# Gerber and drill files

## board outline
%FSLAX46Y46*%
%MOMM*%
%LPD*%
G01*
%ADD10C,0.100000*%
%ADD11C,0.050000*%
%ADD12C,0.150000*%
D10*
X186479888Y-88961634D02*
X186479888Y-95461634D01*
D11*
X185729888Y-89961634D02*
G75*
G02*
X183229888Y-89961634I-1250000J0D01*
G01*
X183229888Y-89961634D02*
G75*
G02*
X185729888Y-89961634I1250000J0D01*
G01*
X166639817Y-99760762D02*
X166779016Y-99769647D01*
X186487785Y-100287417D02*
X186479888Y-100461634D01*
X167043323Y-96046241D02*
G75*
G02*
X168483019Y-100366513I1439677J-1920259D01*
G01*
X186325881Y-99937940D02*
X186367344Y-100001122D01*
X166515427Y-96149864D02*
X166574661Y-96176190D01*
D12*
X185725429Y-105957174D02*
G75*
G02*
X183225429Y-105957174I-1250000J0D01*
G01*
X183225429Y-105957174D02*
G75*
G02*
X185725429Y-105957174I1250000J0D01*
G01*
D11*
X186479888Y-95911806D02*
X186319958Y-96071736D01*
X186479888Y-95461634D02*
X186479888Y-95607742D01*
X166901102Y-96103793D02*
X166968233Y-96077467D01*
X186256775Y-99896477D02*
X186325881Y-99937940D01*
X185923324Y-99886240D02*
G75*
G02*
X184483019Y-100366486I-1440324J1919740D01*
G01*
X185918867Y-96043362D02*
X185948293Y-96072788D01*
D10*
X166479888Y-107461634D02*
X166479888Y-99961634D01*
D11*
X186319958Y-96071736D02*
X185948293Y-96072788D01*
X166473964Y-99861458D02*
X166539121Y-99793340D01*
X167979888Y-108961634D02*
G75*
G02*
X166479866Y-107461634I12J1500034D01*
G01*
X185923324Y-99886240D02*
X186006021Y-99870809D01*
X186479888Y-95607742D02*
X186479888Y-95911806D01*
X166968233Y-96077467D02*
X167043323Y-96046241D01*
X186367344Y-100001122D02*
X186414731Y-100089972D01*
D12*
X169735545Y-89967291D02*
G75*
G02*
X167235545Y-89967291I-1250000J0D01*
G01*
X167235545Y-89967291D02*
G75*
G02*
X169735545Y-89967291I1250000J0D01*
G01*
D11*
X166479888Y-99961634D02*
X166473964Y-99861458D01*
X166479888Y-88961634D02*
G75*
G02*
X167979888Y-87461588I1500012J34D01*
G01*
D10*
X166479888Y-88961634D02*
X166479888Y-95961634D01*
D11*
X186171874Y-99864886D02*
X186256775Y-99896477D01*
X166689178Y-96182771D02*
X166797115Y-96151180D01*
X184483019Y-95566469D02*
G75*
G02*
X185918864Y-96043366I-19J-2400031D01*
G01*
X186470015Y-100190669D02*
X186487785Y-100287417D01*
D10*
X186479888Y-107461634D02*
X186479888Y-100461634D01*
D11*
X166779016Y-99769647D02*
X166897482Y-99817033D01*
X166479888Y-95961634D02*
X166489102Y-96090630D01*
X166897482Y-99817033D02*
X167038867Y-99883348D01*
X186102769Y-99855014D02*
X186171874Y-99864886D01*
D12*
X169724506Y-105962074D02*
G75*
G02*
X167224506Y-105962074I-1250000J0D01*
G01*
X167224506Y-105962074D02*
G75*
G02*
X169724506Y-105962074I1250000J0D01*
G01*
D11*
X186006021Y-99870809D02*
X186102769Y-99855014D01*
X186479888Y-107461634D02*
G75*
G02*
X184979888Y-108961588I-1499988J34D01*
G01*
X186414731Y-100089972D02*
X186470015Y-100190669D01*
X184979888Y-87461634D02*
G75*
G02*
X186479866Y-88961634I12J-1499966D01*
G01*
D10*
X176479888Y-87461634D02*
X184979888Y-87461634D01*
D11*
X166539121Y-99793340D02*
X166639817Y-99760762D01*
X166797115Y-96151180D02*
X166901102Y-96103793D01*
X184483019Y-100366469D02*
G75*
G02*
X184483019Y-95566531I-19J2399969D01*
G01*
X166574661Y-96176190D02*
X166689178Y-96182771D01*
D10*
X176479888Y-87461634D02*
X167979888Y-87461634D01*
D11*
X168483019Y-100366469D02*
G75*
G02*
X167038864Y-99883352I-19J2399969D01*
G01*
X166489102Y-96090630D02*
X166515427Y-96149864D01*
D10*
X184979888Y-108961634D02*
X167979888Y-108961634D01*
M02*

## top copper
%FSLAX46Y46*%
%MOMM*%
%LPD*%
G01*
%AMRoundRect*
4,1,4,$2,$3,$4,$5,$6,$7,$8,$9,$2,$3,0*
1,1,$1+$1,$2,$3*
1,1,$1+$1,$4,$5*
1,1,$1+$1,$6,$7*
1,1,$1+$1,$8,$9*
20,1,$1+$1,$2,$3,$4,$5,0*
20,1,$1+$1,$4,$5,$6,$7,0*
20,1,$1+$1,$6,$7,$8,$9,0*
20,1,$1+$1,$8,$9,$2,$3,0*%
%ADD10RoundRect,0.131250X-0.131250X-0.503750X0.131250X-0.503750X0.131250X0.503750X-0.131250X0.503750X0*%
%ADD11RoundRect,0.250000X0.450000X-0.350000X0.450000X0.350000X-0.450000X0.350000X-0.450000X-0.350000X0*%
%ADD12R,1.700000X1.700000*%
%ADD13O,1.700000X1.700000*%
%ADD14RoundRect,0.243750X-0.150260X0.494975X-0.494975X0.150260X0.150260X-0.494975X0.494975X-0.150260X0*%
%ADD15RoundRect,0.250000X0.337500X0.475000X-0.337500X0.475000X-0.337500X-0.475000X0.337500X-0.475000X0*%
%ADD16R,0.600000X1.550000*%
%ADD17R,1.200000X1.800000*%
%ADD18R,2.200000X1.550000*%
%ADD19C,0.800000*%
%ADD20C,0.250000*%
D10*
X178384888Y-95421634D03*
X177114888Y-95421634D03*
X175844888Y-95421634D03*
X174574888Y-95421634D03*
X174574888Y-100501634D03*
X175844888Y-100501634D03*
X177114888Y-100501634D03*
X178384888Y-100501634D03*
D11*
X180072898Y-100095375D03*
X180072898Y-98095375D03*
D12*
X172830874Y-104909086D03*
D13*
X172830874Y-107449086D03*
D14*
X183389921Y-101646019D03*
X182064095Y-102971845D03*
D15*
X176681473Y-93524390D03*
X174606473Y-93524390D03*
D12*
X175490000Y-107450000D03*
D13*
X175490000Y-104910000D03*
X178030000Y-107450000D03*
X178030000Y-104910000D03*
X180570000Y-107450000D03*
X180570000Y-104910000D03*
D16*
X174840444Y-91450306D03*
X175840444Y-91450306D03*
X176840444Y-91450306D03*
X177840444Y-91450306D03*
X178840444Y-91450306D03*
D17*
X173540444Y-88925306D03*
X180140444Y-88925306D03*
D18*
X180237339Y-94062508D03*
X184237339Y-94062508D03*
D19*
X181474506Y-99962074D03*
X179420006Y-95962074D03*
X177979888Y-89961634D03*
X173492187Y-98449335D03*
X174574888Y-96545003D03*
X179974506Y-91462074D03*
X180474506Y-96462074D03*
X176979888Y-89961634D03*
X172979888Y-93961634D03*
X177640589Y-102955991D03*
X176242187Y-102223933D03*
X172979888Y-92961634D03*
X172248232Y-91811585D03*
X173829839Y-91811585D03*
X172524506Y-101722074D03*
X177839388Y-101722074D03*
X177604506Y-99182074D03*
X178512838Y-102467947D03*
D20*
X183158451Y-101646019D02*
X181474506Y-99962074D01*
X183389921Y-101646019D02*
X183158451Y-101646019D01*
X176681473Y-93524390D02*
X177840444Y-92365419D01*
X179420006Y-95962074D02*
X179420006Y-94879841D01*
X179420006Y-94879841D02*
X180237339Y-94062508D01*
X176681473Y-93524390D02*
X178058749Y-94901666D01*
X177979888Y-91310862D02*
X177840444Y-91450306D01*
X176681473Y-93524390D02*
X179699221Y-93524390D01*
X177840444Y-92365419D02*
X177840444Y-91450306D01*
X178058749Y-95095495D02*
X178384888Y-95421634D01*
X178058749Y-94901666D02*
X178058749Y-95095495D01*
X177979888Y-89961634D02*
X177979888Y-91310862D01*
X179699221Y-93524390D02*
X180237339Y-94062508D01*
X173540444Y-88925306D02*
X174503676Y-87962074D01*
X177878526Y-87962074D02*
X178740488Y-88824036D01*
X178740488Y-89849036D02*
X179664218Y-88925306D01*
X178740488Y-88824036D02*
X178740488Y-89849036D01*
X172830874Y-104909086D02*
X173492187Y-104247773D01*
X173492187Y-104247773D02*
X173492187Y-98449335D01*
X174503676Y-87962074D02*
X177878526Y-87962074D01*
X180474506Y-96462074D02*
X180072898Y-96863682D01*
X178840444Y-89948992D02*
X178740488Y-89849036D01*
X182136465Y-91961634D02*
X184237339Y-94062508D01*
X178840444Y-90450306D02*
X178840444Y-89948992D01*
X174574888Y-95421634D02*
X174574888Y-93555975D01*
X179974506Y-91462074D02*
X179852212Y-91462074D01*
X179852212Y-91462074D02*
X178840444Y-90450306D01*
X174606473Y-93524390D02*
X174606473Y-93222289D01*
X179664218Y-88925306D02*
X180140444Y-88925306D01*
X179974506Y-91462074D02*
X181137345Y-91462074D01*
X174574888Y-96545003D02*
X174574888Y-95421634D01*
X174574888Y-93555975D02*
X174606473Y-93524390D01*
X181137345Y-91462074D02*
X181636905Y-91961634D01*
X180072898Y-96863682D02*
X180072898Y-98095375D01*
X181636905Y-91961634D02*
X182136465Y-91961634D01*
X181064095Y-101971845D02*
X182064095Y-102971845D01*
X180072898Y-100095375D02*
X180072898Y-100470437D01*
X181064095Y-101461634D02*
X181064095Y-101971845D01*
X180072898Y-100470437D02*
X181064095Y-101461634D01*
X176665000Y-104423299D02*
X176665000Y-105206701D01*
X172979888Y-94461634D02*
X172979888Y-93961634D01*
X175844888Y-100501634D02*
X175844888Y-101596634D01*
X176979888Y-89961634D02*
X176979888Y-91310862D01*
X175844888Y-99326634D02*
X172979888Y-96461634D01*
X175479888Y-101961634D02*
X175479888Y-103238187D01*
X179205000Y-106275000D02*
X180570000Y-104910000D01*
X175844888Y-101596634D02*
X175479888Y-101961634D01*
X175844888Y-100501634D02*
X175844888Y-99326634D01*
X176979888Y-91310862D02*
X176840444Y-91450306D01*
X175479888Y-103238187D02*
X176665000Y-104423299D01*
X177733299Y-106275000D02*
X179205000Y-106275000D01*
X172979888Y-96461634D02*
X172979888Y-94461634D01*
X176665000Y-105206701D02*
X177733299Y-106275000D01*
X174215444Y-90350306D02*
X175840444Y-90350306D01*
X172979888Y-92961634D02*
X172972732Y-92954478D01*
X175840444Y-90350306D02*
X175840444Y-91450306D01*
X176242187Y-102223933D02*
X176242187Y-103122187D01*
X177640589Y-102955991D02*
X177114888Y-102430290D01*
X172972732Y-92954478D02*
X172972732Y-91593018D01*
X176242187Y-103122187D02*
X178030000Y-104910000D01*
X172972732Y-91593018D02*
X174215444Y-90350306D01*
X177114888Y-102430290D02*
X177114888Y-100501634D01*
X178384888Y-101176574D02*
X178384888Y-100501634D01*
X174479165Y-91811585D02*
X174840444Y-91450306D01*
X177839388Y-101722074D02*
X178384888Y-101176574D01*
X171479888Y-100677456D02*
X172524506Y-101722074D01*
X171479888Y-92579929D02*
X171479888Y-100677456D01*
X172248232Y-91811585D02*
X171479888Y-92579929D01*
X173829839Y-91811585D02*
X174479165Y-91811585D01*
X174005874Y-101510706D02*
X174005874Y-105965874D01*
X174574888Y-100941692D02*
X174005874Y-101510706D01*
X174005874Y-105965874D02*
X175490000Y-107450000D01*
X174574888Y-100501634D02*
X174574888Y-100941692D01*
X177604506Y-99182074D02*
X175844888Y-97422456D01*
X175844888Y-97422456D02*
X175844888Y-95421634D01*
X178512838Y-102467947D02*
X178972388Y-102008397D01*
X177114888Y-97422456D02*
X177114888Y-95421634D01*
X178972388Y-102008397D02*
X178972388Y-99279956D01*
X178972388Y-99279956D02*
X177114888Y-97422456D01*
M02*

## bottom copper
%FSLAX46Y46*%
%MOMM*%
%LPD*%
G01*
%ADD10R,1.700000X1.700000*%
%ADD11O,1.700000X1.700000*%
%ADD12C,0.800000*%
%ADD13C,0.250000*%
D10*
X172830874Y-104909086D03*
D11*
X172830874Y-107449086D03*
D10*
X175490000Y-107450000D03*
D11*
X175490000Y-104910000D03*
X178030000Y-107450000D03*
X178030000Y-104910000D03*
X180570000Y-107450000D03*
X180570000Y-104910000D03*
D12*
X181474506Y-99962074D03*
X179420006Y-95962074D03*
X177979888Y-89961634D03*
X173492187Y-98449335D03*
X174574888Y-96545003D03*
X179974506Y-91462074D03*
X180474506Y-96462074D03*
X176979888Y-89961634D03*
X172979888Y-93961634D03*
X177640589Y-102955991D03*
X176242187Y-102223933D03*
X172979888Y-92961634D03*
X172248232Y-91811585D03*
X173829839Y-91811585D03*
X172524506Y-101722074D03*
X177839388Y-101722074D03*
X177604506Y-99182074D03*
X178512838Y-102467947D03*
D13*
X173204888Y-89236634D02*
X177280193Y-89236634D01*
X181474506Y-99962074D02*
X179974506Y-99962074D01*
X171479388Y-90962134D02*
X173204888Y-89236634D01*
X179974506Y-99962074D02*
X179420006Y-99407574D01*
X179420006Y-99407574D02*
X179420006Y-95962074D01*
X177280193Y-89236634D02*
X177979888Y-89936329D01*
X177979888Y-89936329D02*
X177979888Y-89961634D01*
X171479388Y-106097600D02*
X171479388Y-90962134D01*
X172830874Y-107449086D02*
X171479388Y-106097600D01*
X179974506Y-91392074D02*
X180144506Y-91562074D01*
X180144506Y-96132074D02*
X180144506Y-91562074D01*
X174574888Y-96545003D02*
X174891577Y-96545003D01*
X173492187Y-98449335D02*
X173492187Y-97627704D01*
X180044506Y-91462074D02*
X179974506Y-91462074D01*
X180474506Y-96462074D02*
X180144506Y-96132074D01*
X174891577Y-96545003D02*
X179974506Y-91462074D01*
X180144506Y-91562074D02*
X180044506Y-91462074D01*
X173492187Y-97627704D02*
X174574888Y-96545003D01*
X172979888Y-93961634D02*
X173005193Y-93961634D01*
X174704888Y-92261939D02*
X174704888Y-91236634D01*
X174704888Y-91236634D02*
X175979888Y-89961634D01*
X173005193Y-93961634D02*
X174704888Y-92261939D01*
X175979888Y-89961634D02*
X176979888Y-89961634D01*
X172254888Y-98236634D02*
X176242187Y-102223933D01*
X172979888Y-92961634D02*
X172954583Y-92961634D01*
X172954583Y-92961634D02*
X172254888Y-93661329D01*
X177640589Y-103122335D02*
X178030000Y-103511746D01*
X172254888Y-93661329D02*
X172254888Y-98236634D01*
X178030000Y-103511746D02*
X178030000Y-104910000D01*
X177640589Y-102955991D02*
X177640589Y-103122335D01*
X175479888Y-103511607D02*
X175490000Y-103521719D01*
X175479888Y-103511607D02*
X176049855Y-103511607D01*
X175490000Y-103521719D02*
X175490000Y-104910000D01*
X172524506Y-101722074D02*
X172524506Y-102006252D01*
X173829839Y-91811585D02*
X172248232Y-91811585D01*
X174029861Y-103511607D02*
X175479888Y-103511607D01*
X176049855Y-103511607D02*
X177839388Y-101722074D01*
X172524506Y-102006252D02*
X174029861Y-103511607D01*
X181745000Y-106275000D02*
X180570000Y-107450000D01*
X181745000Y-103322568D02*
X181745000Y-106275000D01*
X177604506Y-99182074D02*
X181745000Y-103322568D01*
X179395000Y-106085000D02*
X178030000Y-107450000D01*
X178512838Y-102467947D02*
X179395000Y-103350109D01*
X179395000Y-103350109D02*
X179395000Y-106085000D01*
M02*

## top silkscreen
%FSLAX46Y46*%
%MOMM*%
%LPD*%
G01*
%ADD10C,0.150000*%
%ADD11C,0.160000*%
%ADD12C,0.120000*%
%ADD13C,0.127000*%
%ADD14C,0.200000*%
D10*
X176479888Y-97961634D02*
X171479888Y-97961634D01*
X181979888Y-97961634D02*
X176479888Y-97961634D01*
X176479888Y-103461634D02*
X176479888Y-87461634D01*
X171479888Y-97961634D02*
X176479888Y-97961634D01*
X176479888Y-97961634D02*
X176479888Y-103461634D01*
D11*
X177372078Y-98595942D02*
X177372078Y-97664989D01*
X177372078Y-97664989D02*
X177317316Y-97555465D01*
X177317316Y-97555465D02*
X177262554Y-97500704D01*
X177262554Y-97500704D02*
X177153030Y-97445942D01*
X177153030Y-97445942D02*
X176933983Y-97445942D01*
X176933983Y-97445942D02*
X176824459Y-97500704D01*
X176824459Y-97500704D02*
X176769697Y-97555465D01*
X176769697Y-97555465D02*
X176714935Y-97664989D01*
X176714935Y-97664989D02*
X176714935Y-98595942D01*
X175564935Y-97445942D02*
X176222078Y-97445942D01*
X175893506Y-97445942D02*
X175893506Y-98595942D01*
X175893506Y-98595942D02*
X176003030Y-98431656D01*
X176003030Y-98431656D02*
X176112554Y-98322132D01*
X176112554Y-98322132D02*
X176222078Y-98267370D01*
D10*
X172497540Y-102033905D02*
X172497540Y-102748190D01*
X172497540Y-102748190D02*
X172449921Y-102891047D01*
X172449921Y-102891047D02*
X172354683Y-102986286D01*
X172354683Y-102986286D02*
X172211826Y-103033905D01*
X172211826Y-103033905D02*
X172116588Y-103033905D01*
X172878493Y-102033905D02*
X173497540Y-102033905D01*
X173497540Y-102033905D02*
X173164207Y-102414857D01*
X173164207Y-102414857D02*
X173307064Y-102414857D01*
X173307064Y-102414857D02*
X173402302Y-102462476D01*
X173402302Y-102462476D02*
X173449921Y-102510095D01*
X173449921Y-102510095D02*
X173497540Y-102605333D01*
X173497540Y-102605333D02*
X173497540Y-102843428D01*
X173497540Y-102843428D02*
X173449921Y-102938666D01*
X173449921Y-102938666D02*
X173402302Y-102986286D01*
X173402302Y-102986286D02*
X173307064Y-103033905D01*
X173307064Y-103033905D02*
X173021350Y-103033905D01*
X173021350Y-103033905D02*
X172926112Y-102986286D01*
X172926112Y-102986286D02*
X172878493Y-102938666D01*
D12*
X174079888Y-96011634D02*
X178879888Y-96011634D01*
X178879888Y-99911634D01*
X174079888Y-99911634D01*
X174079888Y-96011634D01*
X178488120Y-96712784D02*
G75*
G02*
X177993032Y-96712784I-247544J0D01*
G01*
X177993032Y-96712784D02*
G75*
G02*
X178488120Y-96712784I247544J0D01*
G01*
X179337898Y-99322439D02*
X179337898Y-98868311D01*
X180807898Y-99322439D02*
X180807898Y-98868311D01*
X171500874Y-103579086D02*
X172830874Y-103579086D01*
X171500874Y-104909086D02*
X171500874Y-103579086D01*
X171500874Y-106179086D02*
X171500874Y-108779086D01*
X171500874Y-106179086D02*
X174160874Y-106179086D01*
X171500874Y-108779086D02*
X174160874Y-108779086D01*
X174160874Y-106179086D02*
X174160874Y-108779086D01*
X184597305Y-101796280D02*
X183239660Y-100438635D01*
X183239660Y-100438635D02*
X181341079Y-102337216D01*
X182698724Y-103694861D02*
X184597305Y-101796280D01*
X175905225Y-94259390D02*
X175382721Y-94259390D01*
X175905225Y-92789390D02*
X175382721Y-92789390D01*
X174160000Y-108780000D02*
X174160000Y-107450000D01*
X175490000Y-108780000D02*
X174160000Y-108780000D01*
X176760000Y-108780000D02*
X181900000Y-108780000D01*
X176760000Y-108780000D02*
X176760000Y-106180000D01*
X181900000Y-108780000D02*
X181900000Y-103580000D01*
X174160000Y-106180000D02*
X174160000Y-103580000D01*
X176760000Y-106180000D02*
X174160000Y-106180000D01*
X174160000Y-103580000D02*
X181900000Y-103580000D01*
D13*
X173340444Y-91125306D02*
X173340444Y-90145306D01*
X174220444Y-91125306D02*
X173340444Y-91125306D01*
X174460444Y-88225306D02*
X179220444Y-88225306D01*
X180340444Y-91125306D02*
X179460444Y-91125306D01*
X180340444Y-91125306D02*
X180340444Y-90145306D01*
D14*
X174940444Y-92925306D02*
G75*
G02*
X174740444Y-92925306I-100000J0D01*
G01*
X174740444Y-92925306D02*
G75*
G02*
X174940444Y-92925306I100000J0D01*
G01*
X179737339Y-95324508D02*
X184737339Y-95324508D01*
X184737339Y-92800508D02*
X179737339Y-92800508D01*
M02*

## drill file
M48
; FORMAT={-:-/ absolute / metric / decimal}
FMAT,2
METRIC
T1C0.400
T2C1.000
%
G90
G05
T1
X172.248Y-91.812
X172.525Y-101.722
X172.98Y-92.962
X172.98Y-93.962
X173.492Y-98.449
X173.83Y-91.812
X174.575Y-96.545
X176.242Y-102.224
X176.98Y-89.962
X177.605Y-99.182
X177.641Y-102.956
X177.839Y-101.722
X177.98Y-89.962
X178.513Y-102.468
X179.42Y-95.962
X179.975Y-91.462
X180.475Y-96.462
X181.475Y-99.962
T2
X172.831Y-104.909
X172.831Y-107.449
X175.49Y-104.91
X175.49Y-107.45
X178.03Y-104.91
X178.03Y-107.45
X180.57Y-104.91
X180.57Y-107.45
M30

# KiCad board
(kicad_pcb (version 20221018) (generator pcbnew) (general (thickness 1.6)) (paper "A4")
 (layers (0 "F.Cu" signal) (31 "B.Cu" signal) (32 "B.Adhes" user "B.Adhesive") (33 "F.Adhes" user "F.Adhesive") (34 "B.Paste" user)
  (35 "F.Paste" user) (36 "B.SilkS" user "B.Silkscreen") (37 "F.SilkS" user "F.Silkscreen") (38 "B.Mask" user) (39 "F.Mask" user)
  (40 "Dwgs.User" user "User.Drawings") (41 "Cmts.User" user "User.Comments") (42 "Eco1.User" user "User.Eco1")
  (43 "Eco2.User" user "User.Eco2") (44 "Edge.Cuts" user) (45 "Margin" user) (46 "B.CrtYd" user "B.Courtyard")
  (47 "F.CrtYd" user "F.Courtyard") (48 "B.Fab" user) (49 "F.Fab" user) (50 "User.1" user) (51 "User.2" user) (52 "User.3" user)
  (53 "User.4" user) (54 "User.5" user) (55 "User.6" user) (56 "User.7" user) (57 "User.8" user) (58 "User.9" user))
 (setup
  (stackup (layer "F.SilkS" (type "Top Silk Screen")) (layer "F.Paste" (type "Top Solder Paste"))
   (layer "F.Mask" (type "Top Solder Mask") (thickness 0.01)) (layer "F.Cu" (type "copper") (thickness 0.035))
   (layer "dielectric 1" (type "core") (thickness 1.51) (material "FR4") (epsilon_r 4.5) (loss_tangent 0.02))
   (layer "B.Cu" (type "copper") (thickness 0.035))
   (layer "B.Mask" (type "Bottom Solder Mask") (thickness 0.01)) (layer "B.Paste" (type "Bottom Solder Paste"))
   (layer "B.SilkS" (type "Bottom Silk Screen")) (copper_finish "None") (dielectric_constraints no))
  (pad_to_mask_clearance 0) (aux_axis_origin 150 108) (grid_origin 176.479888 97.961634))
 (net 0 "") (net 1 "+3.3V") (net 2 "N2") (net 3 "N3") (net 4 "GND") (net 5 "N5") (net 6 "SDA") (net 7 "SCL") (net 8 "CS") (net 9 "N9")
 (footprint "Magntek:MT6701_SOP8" (layer "F.Cu") (at 176.479888 97.961634 180)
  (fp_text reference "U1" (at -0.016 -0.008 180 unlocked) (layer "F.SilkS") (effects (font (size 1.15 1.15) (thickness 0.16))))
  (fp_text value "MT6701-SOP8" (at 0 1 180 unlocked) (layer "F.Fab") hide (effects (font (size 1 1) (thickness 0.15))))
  (fp_rect (start -2.4 -1.95) (end 2.4 1.95) (stroke (width 0.12) (type default)) (fill none) (layer "F.SilkS"))
  (fp_circle (center -1.760688 1.24885) (end -1.598307 1.435694) (stroke (width 0.12) (type default)) (fill none) (layer "F.SilkS"))
  (pad "1" smd roundrect (at -1.905 2.54) (size 0.525 1.27) (layers "F.Cu" "F.Paste" "F.Mask") (roundrect_rratio 0.25) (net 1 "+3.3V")
   (thermal_bridge_angle 45))
  (pad "2" smd roundrect (at -0.635 2.54) (size 0.525 1.27) (layers "F.Cu" "F.Paste" "F.Mask") (roundrect_rratio 0.25) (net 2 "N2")
   (thermal_bridge_angle 45))
  (pad "3" smd roundrect (at 0.635 2.54) (size 0.525 1.27) (layers "F.Cu" "F.Paste" "F.Mask") (roundrect_rratio 0.25) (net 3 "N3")
   (thermal_bridge_angle 45))
  (pad "4" smd roundrect (at 1.905 2.54) (size 0.525 1.27) (layers "F.Cu" "F.Paste" "F.Mask") (roundrect_rratio 0.25) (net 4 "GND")
   (thermal_bridge_angle 45))
  (pad "5" smd roundrect (at 1.905 -2.54) (size 0.525 1.27) (layers "F.Cu" "F.Paste" "F.Mask") (roundrect_rratio 0.25) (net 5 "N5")
   (thermal_bridge_angle 45))
  (pad "6" smd roundrect (at 0.635 -2.54) (size 0.525 1.27) (layers "F.Cu" "F.Paste" "F.Mask") (roundrect_rratio 0.25) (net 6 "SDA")
   (thermal_bridge_angle 45))
  (pad "7" smd roundrect (at -0.635 -2.54) (size 0.525 1.27) (layers "F.Cu" "F.Paste" "F.Mask") (roundrect_rratio 0.25) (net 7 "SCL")
   (thermal_bridge_angle 45))
  (pad "8" smd roundrect (at -1.905 -2.54) (size 0.525 1.27) (layers "F.Cu" "F.Paste" "F.Mask") (roundrect_rratio 0.25) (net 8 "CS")
   (thermal_bridge_angle 45)))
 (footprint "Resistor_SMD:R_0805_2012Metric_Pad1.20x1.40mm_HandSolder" (layer "F.Cu") (at 180.072898 99.095375 90)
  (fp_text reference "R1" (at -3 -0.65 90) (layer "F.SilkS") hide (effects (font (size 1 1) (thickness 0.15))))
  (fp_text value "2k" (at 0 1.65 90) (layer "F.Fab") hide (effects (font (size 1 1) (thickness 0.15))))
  (fp_line (start -0.227064 -0.735) (end 0.227064 -0.735) (stroke (width 0.12) (type solid)) (layer "F.SilkS"))
  (fp_line (start -0.227064 0.735) (end 0.227064 0.735) (stroke (width 0.12) (type solid)) (layer "F.SilkS"))
  (pad "1" smd roundrect (at -1 0 90) (size 1.2 1.4) (layers "F.Cu" "F.Paste" "F.Mask") (roundrect_rratio 0.208333) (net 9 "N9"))
  (pad "2" smd roundrect (at 1 0 90) (size 1.2 1.4) (layers "F.Cu" "F.Paste" "F.Mask") (roundrect_rratio 0.208333) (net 4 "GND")))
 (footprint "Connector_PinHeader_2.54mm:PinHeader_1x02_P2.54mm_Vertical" (layer "F.Cu") (at 172.830874 104.909086)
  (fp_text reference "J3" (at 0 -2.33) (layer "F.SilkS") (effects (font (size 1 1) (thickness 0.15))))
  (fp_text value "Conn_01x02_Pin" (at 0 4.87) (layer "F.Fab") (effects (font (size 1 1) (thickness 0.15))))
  (fp_line (start -1.33 -1.33) (end 0 -1.33) (stroke (width 0.12) (type solid)) (layer "F.SilkS"))
  (fp_line (start -1.33 0) (end -1.33 -1.33) (stroke (width 0.12) (type solid)) (layer "F.SilkS"))
  (fp_line (start -1.33 1.27) (end -1.33 3.87) (stroke (width 0.12) (type solid)) (layer "F.SilkS"))
  (fp_line (start -1.33 1.27) (end 1.33 1.27) (stroke (width 0.12) (type solid)) (layer "F.SilkS"))
  (fp_line (start -1.33 3.87) (end 1.33 3.87) (stroke (width 0.12) (type solid)) (layer "F.SilkS"))
  (fp_line (start 1.33 1.27) (end 1.33 3.87) (stroke (width 0.12) (type solid)) (layer "F.SilkS"))
  (pad "1" thru_hole rect (at 0 0) (size 1.7 1.7) (drill 1) (layers "*.Cu" "*.Mask") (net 4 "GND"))
  (pad "2" thru_hole oval (at 0 2.54) (size 1.7 1.7) (drill 1) (layers "*.Cu" "*.Mask") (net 1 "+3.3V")))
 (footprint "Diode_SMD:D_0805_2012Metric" (layer "F.Cu") (at 182.727008 102.308932 -135)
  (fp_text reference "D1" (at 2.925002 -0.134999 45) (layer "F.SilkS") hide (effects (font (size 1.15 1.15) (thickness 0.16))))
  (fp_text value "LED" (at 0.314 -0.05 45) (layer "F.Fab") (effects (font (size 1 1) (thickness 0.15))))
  (fp_line (start -1.685 -0.96) (end -1.685 0.96) (stroke (width 0.12) (type solid)) (layer "F.SilkS"))
  (fp_line (start -1.685 0.96) (end 1 0.96) (stroke (width 0.12) (type solid)) (layer "F.SilkS"))
  (fp_line (start 1 -0.96) (end -1.685 -0.96) (stroke (width 0.12) (type solid)) (layer "F.SilkS"))
  (pad "1" smd roundrect (at -0.9375 0 225) (size 0.975 1.4) (layers "F.Cu" "F.Paste" "F.Mask") (roundrect_rratio 0.25) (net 1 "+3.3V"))
  (pad "2" smd roundrect (at 0.9375 0 225) (size 0.975 1.4) (layers "F.Cu" "F.Paste" "F.Mask") (roundrect_rratio 0.25) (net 9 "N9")))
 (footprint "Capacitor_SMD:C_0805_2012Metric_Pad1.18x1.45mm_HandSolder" (layer "F.Cu") (at 175.643973 93.52439 180)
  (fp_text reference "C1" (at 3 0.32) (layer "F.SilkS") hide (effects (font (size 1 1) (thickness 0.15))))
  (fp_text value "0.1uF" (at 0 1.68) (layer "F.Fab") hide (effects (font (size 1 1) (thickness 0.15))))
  (fp_line (start -0.261252 -0.735) (end 0.261252 -0.735) (stroke (width 0.12) (type solid)) (layer "F.SilkS"))
  (fp_line (start -0.261252 0.735) (end 0.261252 0.735) (stroke (width 0.12) (type solid)) (layer "F.SilkS"))
  (pad "1" smd roundrect (at -1.0375 0 180) (size 1.175 1.45) (layers "F.Cu" "F.Paste" "F.Mask") (roundrect_rratio 0.212766) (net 1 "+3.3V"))
  (pad "2" smd roundrect (at 1.0375 0 180) (size 1.175 1.45) (layers "F.Cu" "F.Paste" "F.Mask") (roundrect_rratio 0.212766) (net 4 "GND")))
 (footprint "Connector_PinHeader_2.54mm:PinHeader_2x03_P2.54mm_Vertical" (layer "F.Cu") (at 175.49 107.45 90)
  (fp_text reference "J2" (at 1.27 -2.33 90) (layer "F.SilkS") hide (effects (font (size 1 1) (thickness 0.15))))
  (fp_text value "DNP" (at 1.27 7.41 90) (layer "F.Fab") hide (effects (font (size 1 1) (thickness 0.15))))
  (fp_line (start -1.33 -1.33) (end 0 -1.33) (stroke (width 0.12) (type solid)) (layer "F.SilkS"))
  (fp_line (start -1.33 0) (end -1.33 -1.33) (stroke (width 0.12) (type solid)) (layer "F.SilkS"))
  (fp_line (start -1.33 1.27) (end -1.33 6.41) (stroke (width 0.12) (type solid)) (layer "F.SilkS"))
  (fp_line (start -1.33 1.27) (end 1.27 1.27) (stroke (width 0.12) (type solid)) (layer "F.SilkS"))
  (fp_line (start -1.33 6.41) (end 3.87 6.41) (stroke (width 0.12) (type solid)) (layer "F.SilkS"))
  (fp_line (start 1.27 -1.33) (end 3.87 -1.33) (stroke (width 0.12) (type solid)) (layer "F.SilkS"))
  (fp_line (start 1.27 1.27) (end 1.27 -1.33) (stroke (width 0.12) (type solid)) (layer "F.SilkS"))
  (fp_line (start 3.87 -1.33) (end 3.87 6.41) (stroke (width 0.12) (type solid)) (layer "F.SilkS"))
  (pad "1" thru_hole rect (at 0 0 90) (size 1.7 1.7) (drill 1) (layers "*.Cu" "*.Mask") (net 5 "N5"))
  (pad "2" thru_hole oval (at 2.54 0 90) (size 1.7 1.7) (drill 1) (layers "*.Cu" "*.Mask") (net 8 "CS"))
  (pad "3" thru_hole oval (at 0 2.54 90) (size 1.7 1.7) (drill 1) (layers "*.Cu" "*.Mask") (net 2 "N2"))
  (pad "4" thru_hole oval (at 2.54 2.54 90) (size 1.7 1.7) (drill 1) (layers "*.Cu" "*.Mask") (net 7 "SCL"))
  (pad "5" thru_hole oval (at 0 5.08 90) (size 1.7 1.7) (drill 1) (layers "*.Cu" "*.Mask") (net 3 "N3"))
  (pad "6" thru_hole oval (at 2.54 5.08 90) (size 1.7 1.7) (drill 1) (layers "*.Cu" "*.Mask") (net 6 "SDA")))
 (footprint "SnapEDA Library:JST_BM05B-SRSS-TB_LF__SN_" (layer "F.Cu") (at 176.840444 88.925306)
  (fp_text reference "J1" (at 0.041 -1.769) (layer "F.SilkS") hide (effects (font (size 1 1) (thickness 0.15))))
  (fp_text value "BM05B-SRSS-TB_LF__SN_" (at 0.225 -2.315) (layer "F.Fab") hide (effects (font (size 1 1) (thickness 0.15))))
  (fp_line (start -3.5 2.2) (end -3.5 1.22) (stroke (width 0.127) (type solid)) (layer "F.SilkS"))
  (fp_line (start -2.62 2.2) (end -3.5 2.2) (stroke (width 0.127) (type solid)) (layer "F.SilkS"))
  (fp_line (start -2.38 -0.7) (end 2.38 -0.7) (stroke (width 0.127) (type solid)) (layer "F.SilkS"))
  (fp_line (start 3.5 2.2) (end 2.62 2.2) (stroke (width 0.127) (type solid)) (layer "F.SilkS"))
  (fp_line (start 3.5 2.2) (end 3.5 1.22) (stroke (width 0.127) (type solid)) (layer "F.SilkS"))
  (fp_circle (center -2 4) (end -1.9 4) (stroke (width 0.2) (type solid)) (fill none) (layer "F.SilkS"))
  (pad "1" smd rect (at -2 2.525) (size 0.6 1.55) (layers "F.Cu" "F.Paste" "F.Mask") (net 8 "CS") (solder_mask_margin 0.102))
  (pad "2" smd rect (at -1 2.525) (size 0.6 1.55) (layers "F.Cu" "F.Paste" "F.Mask") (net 7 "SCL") (solder_mask_margin 0.102))
  (pad "3" smd rect (at 0 2.525) (size 0.6 1.55) (layers "F.Cu" "F.Paste" "F.Mask") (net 6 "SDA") (solder_mask_margin 0.102))
  (pad "4" smd rect (at 1 2.525) (size 0.6 1.55) (layers "F.Cu" "F.Paste" "F.Mask") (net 1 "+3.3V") (solder_mask_margin 0.102))
  (pad "5" smd rect (at 2 2.525) (size 0.6 1.55) (layers "F.Cu" "F.Paste" "F.Mask") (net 4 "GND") (solder_mask_margin 0.102))
  (pad "S1" smd rect (at -3.3 0) (size 1.2 1.8) (layers "F.Cu" "F.Paste" "F.Mask") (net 4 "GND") (solder_mask_margin 0.102))
  (pad "S2" smd rect (at 3.3 0) (size 1.2 1.8) (layers "F.Cu" "F.Paste" "F.Mask") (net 4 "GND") (solder_mask_margin 0.102)))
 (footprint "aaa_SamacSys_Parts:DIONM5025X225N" (layer "F.Cu") (at 182.237339 94.062508)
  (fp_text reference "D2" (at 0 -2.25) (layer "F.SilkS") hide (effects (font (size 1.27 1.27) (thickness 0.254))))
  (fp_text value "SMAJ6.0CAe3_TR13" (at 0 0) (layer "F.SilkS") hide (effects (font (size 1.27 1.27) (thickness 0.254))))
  (fp_line (start -2.5 1.262) (end 2.5 1.262) (stroke (width 0.2) (type solid)) (layer "F.SilkS"))
  (fp_line (start 2.5 -1.262) (end -2.5 -1.262) (stroke (width 0.2) (type solid)) (layer "F.SilkS"))
  (pad "1" smd rect (at -2 0 90) (size 1.55 2.2) (layers "F.Cu" "F.Paste" "F.Mask") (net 1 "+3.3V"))
  (pad "2" smd rect (at 2 0 90) (size 1.55 2.2) (layers "F.Cu" "F.Paste" "F.Mask") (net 4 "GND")))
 (gr_line (start 176.479888 97.961634) (end 171.479888 97.961634) (stroke (width 0.15) (type default)) (layer "F.SilkS"))
 (gr_line (start 181.979888 97.961634) (end 176.479888 97.961634) (stroke (width 0.15) (type default)) (layer "F.SilkS"))
 (gr_line (start 176.479888 103.461634) (end 176.479888 87.461634) (stroke (width 0.15) (type default)) (layer "F.SilkS"))
 (gr_line (start 171.479888 97.961634) (end 176.479888 97.961634) (stroke (width 0.15) (type default)) (layer "F.SilkS"))
 (gr_line (start 176.479888 97.961634) (end 176.479888 103.461634) (stroke (width 0.15) (type default)) (layer "F.SilkS"))
 (gr_line (start 186.479888 88.961634) (end 186.479888 95.461634) (stroke (width 0.1) (type default)) (layer "Edge.Cuts"))
 (gr_circle (center 184.479888 89.961634) (end 185.729888 89.961634) (stroke (width 0.05) (type default)) (fill none) (layer "Edge.Cuts"))
 (gr_line (start 166.639817 99.760762) (end 166.779016 99.769647) (stroke (width 0.05) (type default)) (layer "Edge.Cuts"))
 (gr_line (start 186.487785 100.287417) (end 186.479888 100.461634) (stroke (width 0.05) (type default)) (layer "Edge.Cuts"))
 (gr_arc (start 167.043323 96.046241) (mid 170.759919 97.207703) (end 168.483019 100.366469) (stroke (width 0.05) (type default))
  (layer "Edge.Cuts"))
 (gr_line (start 186.325881 99.93794) (end 186.367344 100.001122) (stroke (width 0.05) (type default)) (layer "Edge.Cuts"))
 (gr_line (start 166.515427 96.149864) (end 166.574661 96.17619) (stroke (width 0.05) (type default)) (layer "Edge.Cuts"))
 (gr_circle (center 184.475429 105.957174) (end 185.725429 105.957174) (stroke (width 0.15) (type default)) (fill none) (layer "Edge.Cuts"))
 (gr_line (start 186.479888 95.911806) (end 186.319958 96.071736) (stroke (width 0.05) (type default)) (layer "Edge.Cuts"))
 (gr_line (start 186.479888 95.461634) (end 186.479888 95.607742) (stroke (width 0.05) (type default)) (layer "Edge.Cuts"))
 (gr_line (start 166.901102 96.103793) (end 166.968233 96.077467) (stroke (width 0.05) (type default)) (layer "Edge.Cuts"))
 (gr_line (start 186.256775 99.896477) (end 186.325881 99.93794) (stroke (width 0.05) (type default)) (layer "Edge.Cuts"))
 (gr_arc (start 185.923324 99.88624) (mid 185.242146 100.243248) (end 184.483019 100.366469) (stroke (width 0.05) (type default))
  (layer "Edge.Cuts"))
 (gr_line (start 185.918867 96.043362) (end 185.948293 96.072788) (stroke (width 0.05) (type default)) (layer "Edge.Cuts"))
 (gr_line (start 166.479888 107.461634) (end 166.479888 99.961634) (stroke (width 0.1) (type default)) (layer "Edge.Cuts"))
 (gr_line (start 186.319958 96.071736) (end 185.948293 96.072788) (stroke (width 0.05) (type default)) (layer "Edge.Cuts"))
 (gr_line (start 166.473964 99.861458) (end 166.539121 99.79334) (stroke (width 0.05) (type default)) (layer "Edge.Cuts"))
 (gr_arc (start 167.979888 108.961634) (mid 166.919228 108.522294) (end 166.479888 107.461634) (stroke (width 0.05) (type default))
  (layer "Edge.Cuts"))
 (gr_line (start 185.923324 99.88624) (end 186.006021 99.870809) (stroke (width 0.05) (type default)) (layer "Edge.Cuts"))
 (gr_line (start 186.479888 95.607742) (end 186.479888 95.911806) (stroke (width 0.05) (type default)) (layer "Edge.Cuts"))
 (gr_line (start 166.968233 96.077467) (end 167.043323 96.046241) (stroke (width 0.05) (type default)) (layer "Edge.Cuts"))
 (gr_line (start 186.367344 100.001122) (end 186.414731 100.089972) (stroke (width 0.05) (type default)) (layer "Edge.Cuts"))
 (gr_circle (center 168.485545 89.967291) (end 169.735545 89.967291) (stroke (width 0.15) (type default)) (fill none) (layer "Edge.Cuts"))
 (gr_line (start 166.479888 99.961634) (end 166.473964 99.861458) (stroke (width 0.05) (type default)) (layer "Edge.Cuts"))
 (gr_arc (start 166.479888 88.961634) (mid 166.919228 87.900974) (end 167.979888 87.461634) (stroke (width 0.05) (type default))
  (layer "Edge.Cuts"))
 (gr_line (start 166.479888 88.961634) (end 166.479888 95.961634) (stroke (width 0.1) (type default)) (layer "Edge.Cuts"))
 (gr_line (start 186.171874 99.864886) (end 186.256775 99.896477) (stroke (width 0.05) (type default)) (layer "Edge.Cuts"))
 (gr_line (start 166.689178 96.182771) (end 166.797115 96.15118) (stroke (width 0.05) (type default)) (layer "Edge.Cuts"))
 (gr_arc (start 184.483019 95.566469) (mid 185.239505 95.68881) (end 185.918867 96.043362) (stroke (width 0.05) (type default))
  (layer "Edge.Cuts"))
 (gr_line (start 186.470015 100.190669) (end 186.487785 100.287417) (stroke (width 0.05) (type default)) (layer "Edge.Cuts"))
 (gr_line (start 186.479888 107.461634) (end 186.479888 100.461634) (stroke (width 0.1) (type default)) (layer "Edge.Cuts"))
 (gr_line (start 166.779016 99.769647) (end 166.897482 99.817033) (stroke (width 0.05) (type default)) (layer "Edge.Cuts"))
 (gr_line (start 166.479888 95.961634) (end 166.489102 96.09063) (stroke (width 0.05) (type default)) (layer "Edge.Cuts"))
 (gr_line (start 166.897482 99.817033) (end 167.038867 99.883348) (stroke (width 0.05) (type default)) (layer "Edge.Cuts"))
 (gr_line (start 186.102769 99.855014) (end 186.171874 99.864886) (stroke (width 0.05) (type default)) (layer "Edge.Cuts"))
 (gr_circle (center 168.474506 105.962074) (end 169.724506 105.962074) (stroke (width 0.15) (type default)) (fill none) (layer "Edge.Cuts"))
 (gr_line (start 186.006021 99.870809) (end 186.102769 99.855014) (stroke (width 0.05) (type default)) (layer "Edge.Cuts"))
 (gr_arc (start 186.479888 107.461634) (mid 186.040548 108.522294) (end 184.979888 108.961634) (stroke (width 0.05) (type default))
  (layer "Edge.Cuts"))
 (gr_line (start 186.414731 100.089972) (end 186.470015 100.190669) (stroke (width 0.05) (type default)) (layer "Edge.Cuts"))
 (gr_arc (start 184.979888 87.461634) (mid 186.040548 87.900974) (end 186.479888 88.961634) (stroke (width 0.05) (type default))
  (layer "Edge.Cuts"))
 (gr_line (start 176.479888 87.461634) (end 184.979888 87.461634) (stroke (width 0.1) (type default)) (layer "Edge.Cuts"))
 (gr_line (start 166.539121 99.79334) (end 166.639817 99.760762) (stroke (width 0.05) (type default)) (layer "Edge.Cuts"))
 (gr_line (start 166.797115 96.15118) (end 166.901102 96.103793) (stroke (width 0.05) (type default)) (layer "Edge.Cuts"))
 (gr_arc (start 184.483019 100.366469) (mid 182.083019 97.966469) (end 184.483019 95.566469) (stroke (width 0.05) (type default))
  (layer "Edge.Cuts"))
 (gr_line (start 166.574661 96.17619) (end 166.689178 96.182771) (stroke (width 0.05) (type default)) (layer "Edge.Cuts"))
 (gr_line (start 176.479888 87.461634) (end 167.979888 87.461634) (stroke (width 0.1) (type default)) (layer "Edge.Cuts"))
 (gr_arc (start 168.483019 100.366469) (mid 167.721609 100.242486) (end 167.038867 99.883348) (stroke (width 0.05) (type default))
  (layer "Edge.Cuts"))
 (gr_line (start 166.489102 96.09063) (end 166.515427 96.149864) (stroke (width 0.05) (type default)) (layer "Edge.Cuts"))
 (gr_line (start 184.979888 108.961634) (end 167.979888 108.961634) (stroke (width 0.1) (type default)) (layer "Edge.Cuts"))
 (segment (start 183.158451 101.646019) (end 181.474506 99.962074) (width 0.25) (layer "F.Cu") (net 1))
 (segment (start 183.389921 101.646019) (end 183.158451 101.646019) (width 0.25) (layer "F.Cu") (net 1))
 (segment (start 176.681473 93.52439) (end 177.840444 92.365419) (width 0.25) (layer "F.Cu") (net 1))
 (segment (start 179.420006 95.962074) (end 179.420006 94.879841) (width 0.25) (layer "F.Cu") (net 1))
 (segment (start 179.420006 94.879841) (end 180.237339 94.062508) (width 0.25) (layer "F.Cu") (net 1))
 (segment (start 176.681473 93.52439) (end 178.058749 94.901666) (width 0.25) (layer "F.Cu") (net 1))
 (segment (start 177.979888 91.310862) (end 177.840444 91.450306) (width 0.25) (layer "F.Cu") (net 1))
 (segment (start 176.681473 93.52439) (end 179.699221 93.52439) (width 0.25) (layer "F.Cu") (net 1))
 (segment (start 177.840444 92.365419) (end 177.840444 91.450306) (width 0.25) (layer "F.Cu") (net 1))
 (segment (start 178.058749 95.095495) (end 178.384888 95.421634) (width 0.25) (layer "F.Cu") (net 1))
 (segment (start 178.058749 94.901666) (end 178.058749 95.095495) (width 0.25) (layer "F.Cu") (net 1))
 (segment (start 177.979888 89.961634) (end 177.979888 91.310862) (width 0.25) (layer "F.Cu") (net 1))
 (segment (start 179.699221 93.52439) (end 180.237339 94.062508) (width 0.25) (layer "F.Cu") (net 1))
 (via (at 181.474506 99.962074) (size 0.8) (drill 0.4) (layers "F.Cu" "B.Cu") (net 1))
 (via (at 179.420006 95.962074) (size 0.8) (drill 0.4) (layers "F.Cu" "B.Cu") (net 1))
 (via (at 177.979888 89.961634) (size 0.8) (drill 0.4) (layers "F.Cu" "B.Cu") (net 1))
 (segment (start 173.204888 89.236634) (end 177.280193 89.236634) (width 0.25) (layer "B.Cu") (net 1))
 (segment (start 181.474506 99.962074) (end 179.974506 99.962074) (width 0.25) (layer "B.Cu") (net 1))
 (segment (start 171.479388 90.962134) (end 173.204888 89.236634) (width 0.25) (layer "B.Cu") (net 1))
 (segment (start 179.974506 99.962074) (end 179.420006 99.407574) (width 0.25) (layer "B.Cu") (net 1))
 (segment (start 179.420006 99.407574) (end 179.420006 95.962074) (width 0.25) (layer "B.Cu") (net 1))
 (segment (start 177.280193 89.236634) (end 177.979888 89.936329) (width 0.25) (layer "B.Cu") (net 1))
 (segment (start 177.979888 89.936329) (end 177.979888 89.961634) (width 0.25) (layer "B.Cu") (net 1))
 (segment (start 171.479388 106.0976) (end 171.479388 90.962134) (width 0.25) (layer "B.Cu") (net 1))
 (segment (start 172.830874 107.449086) (end 171.479388 106.0976) (width 0.25) (layer "B.Cu") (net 1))
 (segment (start 173.540444 88.925306) (end 174.503676 87.962074) (width 0.25) (layer "F.Cu") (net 4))
 (segment (start 177.878526 87.962074) (end 178.740488 88.824036) (width 0.25) (layer "F.Cu") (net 4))
 (segment (start 178.740488 89.849036) (end 179.664218 88.925306) (width 0.25) (layer "F.Cu") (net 4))
 (segment (start 178.740488 88.824036) (end 178.740488 89.849036) (width 0.25) (layer "F.Cu") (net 4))
 (segment (start 172.830874 104.909086) (end 173.492187 104.247773) (width 0.25) (layer "F.Cu") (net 4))
 (segment (start 173.492187 104.247773) (end 173.492187 98.449335) (width 0.25) (layer "F.Cu") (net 4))
 (segment (start 174.503676 87.962074) (end 177.878526 87.962074) (width 0.25) (layer "F.Cu") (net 4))
 (segment (start 180.474506 96.462074) (end 180.072898 96.863682) (width 0.25) (layer "F.Cu") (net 4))
 (segment (start 178.840444 89.948992) (end 178.740488 89.849036) (width 0.25) (layer "F.Cu") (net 4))
 (segment (start 182.136465 91.961634) (end 184.237339 94.062508) (width 0.25) (layer "F.Cu") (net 4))
 (segment (start 178.840444 90.450306) (end 178.840444 89.948992) (width 0.25) (layer "F.Cu") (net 4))
 (segment (start 174.574888 95.421634) (end 174.574888 93.555975) (width 0.25) (layer "F.Cu") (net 4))
 (segment (start 179.974506 91.462074) (end 179.852212 91.462074) (width 0.25) (layer "F.Cu") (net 4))
 (segment (start 179.852212 91.462074) (end 178.840444 90.450306) (width 0.25) (layer "F.Cu") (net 4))
 (segment (start 174.606473 93.52439) (end 174.606473 93.222289) (width 0.25) (layer "F.Cu") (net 4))
 (segment (start 179.664218 88.925306) (end 180.140444 88.925306) (width 0.25) (layer "F.Cu") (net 4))
 (segment (start 179.974506 91.462074) (end 181.137345 91.462074) (width 0.25) (layer "F.Cu") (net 4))
 (segment (start 174.574888 96.545003) (end 174.574888 95.421634) (width 0.25) (layer "F.Cu") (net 4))
 (segment (start 174.574888 93.555975) (end 174.606473 93.52439) (width 0.25) (layer "F.Cu") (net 4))
 (segment (start 181.137345 91.462074) (end 181.636905 91.961634) (width 0.25) (layer "F.Cu") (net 4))
 (segment (start 180.072898 96.863682) (end 180.072898 98.095375) (width 0.25) (layer "F.Cu") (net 4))
 (segment (start 181.636905 91.961634) (end 182.136465 91.961634) (width 0.25) (layer "F.Cu") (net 4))
 (via (at 173.492187 98.449335) (size 0.8) (drill 0.4) (layers "F.Cu" "B.Cu") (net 4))
 (via (at 174.574888 96.545003) (size 0.8) (drill 0.4) (layers "F.Cu" "B.Cu") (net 4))
 (via (at 179.974506 91.462074) (size 0.8) (drill 0.4) (layers "F.Cu" "B.Cu") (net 4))
 (via (at 180.474506 96.462074) (size 0.8) (drill 0.4) (layers "F.Cu" "B.Cu") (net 4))
 (segment (start 179.974506 91.392074) (end 180.144506 91.562074) (width 0.25) (layer "B.Cu") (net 4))
 (segment (start 180.144506 96.132074) (end 180.144506 91.562074) (width 0.25) (layer "B.Cu") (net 4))
 (segment (start 174.574888 96.545003) (end 174.891577 96.545003) (width 0.25) (layer "B.Cu") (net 4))
 (segment (start 173.492187 98.449335) (end 173.492187 97.627704) (width 0.25) (layer "B.Cu") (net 4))
 (segment (start 180.044506 91.462074) (end 179.974506 91.462074) (width 0.25) (layer "B.Cu") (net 4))
 (segment (start 180.474506 96.462074) (end 180.144506 96.132074) (width 0.25) (layer "B.Cu") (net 4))
 (segment (start 174.891577 96.545003) (end 179.974506 91.462074) (width 0.25) (layer "B.Cu") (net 4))
 (segment (start 180.144506 91.562074) (end 180.044506 91.462074) (width 0.25) (layer "B.Cu") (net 4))
 (segment (start 173.492187 97.627704) (end 174.574888 96.545003) (width 0.25) (layer "B.Cu") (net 4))
 (segment (start 181.064095 101.971845) (end 182.064095 102.971845) (width 0.25) (layer "F.Cu") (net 9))
 (segment (start 180.072898 100.095375) (end 180.072898 100.470437) (width 0.25) (layer "F.Cu") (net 9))
 (segment (start 181.064095 101.461634) (end 181.064095 101.971845) (width 0.25) (layer "F.Cu") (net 9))
 (segment (start 180.072898 100.470437) (end 181.064095 101.461634) (width 0.25) (layer "F.Cu") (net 9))
 (segment (start 176.665 104.423299) (end 176.665 105.206701) (width 0.25) (layer "F.Cu") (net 6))
 (segment (start 172.979888 94.461634) (end 172.979888 93.961634) (width 0.25) (layer "F.Cu") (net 6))
 (segment (start 175.844888 100.501634) (end 175.844888 101.596634) (width 0.25) (layer "F.Cu") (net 6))
 (segment (start 176.979888 89.961634) (end 176.979888 91.310862) (width 0.25) (layer "F.Cu") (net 6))
 (segment (start 175.844888 99.326634) (end 172.979888 96.461634) (width 0.25) (layer "F.Cu") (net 6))
 (segment (start 175.479888 101.961634) (end 175.479888 103.238187) (width 0.25) (layer "F.Cu") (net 6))
 (segment (start 179.205 106.275) (end 180.57 104.91) (width 0.25) (layer "F.Cu") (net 6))
 (segment (start 175.844888 101.596634) (end 175.479888 101.961634) (width 0.25) (layer "F.Cu") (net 6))
 (segment (start 175.844888 100.501634) (end 175.844888 99.326634) (width 0.25) (layer "F.Cu") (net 6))
 (segment (start 176.979888 91.310862) (end 176.840444 91.450306) (width 0.25) (layer "F.Cu") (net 6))
 (segment (start 175.479888 103.238187) (end 176.665 104.423299) (width 0.25) (layer "F.Cu") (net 6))
 (segment (start 177.733299 106.275) (end 179.205 106.275) (width 0.25) (layer "F.Cu") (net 6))
 (segment (start 172.979888 96.461634) (end 172.979888 94.461634) (width 0.25) (layer "F.Cu") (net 6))
 (segment (start 176.665 105.206701) (end 177.733299 106.275) (width 0.25) (layer "F.Cu") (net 6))
 (via (at 176.979888 89.961634) (size 0.8) (drill 0.4) (layers "F.Cu" "B.Cu") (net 6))
 (via (at 172.979888 93.961634) (size 0.8) (drill 0.4) (layers "F.Cu" "B.Cu") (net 6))
 (segment (start 172.979888 93.961634) (end 173.005193 93.961634) (width 0.25) (layer "B.Cu") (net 6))
 (segment (start 174.704888 92.261939) (end 174.704888 91.236634) (width 0.25) (layer "B.Cu") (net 6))
 (segment (start 174.704888 91.236634) (end 175.979888 89.961634) (width 0.25) (layer "B.Cu") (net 6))
 (segment (start 173.005193 93.961634) (end 174.704888 92.261939) (width 0.25) (layer "B.Cu") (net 6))
 (segment (start 175.979888 89.961634) (end 176.979888 89.961634) (width 0.25) (layer "B.Cu") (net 6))
 (segment (start 174.215444 90.350306) (end 175.840444 90.350306) (width 0.25) (layer "F.Cu") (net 7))
 (segment (start 172.979888 92.961634) (end 172.972732 92.954478) (width 0.25) (layer "F.Cu") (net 7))
 (segment (start 175.840444 90.350306) (end 175.840444 91.450306) (width 0.25) (layer "F.Cu") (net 7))
 (segment (start 176.242187 102.223933) (end 176.242187 103.122187) (width 0.25) (layer "F.Cu") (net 7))
 (segment (start 177.640589 102.955991) (end 177.114888 102.43029) (width 0.25) (layer "F.Cu") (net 7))
 (segment (start 172.972732 92.954478) (end 172.972732 91.593018) (width 0.25) (layer "F.Cu") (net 7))
 (segment (start 176.242187 103.122187) (end 178.03 104.91) (width 0.25) (layer "F.Cu") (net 7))
 (segment (start 172.972732 91.593018) (end 174.215444 90.350306) (width 0.25) (layer "F.Cu") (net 7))
 (segment (start 177.114888 102.43029) (end 177.114888 100.501634) (width 0.25) (layer "F.Cu") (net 7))
 (via (at 177.640589 102.955991) (size 0.8) (drill 0.4) (layers "F.Cu" "B.Cu") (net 7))
 (via (at 176.242187 102.223933) (size 0.8) (drill 0.4) (layers "F.Cu" "B.Cu") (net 7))
 (via (at 172.979888 92.961634) (size 0.8) (drill 0.4) (layers "F.Cu" "B.Cu") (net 7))
 (segment (start 172.254888 98.236634) (end 176.242187 102.223933) (width 0.25) (layer "B.Cu") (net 7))
 (segment (start 172.979888 92.961634) (end 172.954583 92.961634) (width 0.25) (layer "B.Cu") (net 7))
 (segment (start 172.954583 92.961634) (end 172.254888 93.661329) (width 0.25) (layer "B.Cu") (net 7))
 (segment (start 177.640589 103.122335) (end 178.03 103.511746) (width 0.25) (layer "B.Cu") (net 7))
 (segment (start 172.254888 93.661329) (end 172.254888 98.236634) (width 0.25) (layer "B.Cu") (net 7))
 (segment (start 178.03 103.511746) (end 178.03 104.91) (width 0.25) (layer "B.Cu") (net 7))
 (segment (start 177.640589 102.955991) (end 177.640589 103.122335) (width 0.25) (layer "B.Cu") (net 7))
 (segment (start 178.384888 101.176574) (end 178.384888 100.501634) (width 0.25) (layer "F.Cu") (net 8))
 (segment (start 174.479165 91.811585) (end 174.840444 91.450306) (width 0.25) (layer "F.Cu") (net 8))
 (segment (start 177.839388 101.722074) (end 178.384888 101.176574) (width 0.25) (layer "F.Cu") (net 8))
 (segment (start 171.479888 100.677456) (end 172.524506 101.722074) (width 0.25) (layer "F.Cu") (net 8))
 (segment (start 171.479888 92.579929) (end 171.479888 100.677456) (width 0.25) (layer "F.Cu") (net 8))
 (segment (start 172.248232 91.811585) (end 171.479888 92.579929) (width 0.25) (layer "F.Cu") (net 8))
 (segment (start 173.829839 91.811585) (end 174.479165 91.811585) (width 0.25) (layer "F.Cu") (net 8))
 (via (at 172.248232 91.811585) (size 0.8) (drill 0.4) (layers "F.Cu" "B.Cu") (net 8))
 (via (at 173.829839 91.811585) (size 0.8) (drill 0.4) (layers "F.Cu" "B.Cu") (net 8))
 (via (at 172.524506 101.722074) (size 0.8) (drill 0.4) (layers "F.Cu" "B.Cu") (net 8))
 (via (at 177.839388 101.722074) (size 0.8) (drill 0.4) (layers "F.Cu" "B.Cu") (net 8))
 (segment (start 175.479888 103.511607) (end 175.49 103.521719) (width 0.25) (layer "B.Cu") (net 8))
 (segment (start 175.479888 103.511607) (end 176.049855 103.511607) (width 0.25) (layer "B.Cu") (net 8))
 (segment (start 175.49 103.521719) (end 175.49 104.91) (width 0.25) (layer "B.Cu") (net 8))
 (segment (start 172.524506 101.722074) (end 172.524506 102.006252) (width 0.25) (layer "B.Cu") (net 8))
 (segment (start 173.829839 91.811585) (end 172.248232 91.811585) (width 0.25) (layer "B.Cu") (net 8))
 (segment (start 174.029861 103.511607) (end 175.479888 103.511607) (width 0.25) (layer "B.Cu") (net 8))
 (segment (start 176.049855 103.511607) (end 177.839388 101.722074) (width 0.25) (layer "B.Cu") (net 8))
 (segment (start 172.524506 102.006252) (end 174.029861 103.511607) (width 0.25) (layer "B.Cu") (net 8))
 (segment (start 174.005874 101.510706) (end 174.005874 105.965874) (width 0.25) (layer "F.Cu") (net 5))
 (segment (start 174.574888 100.941692) (end 174.005874 101.510706) (width 0.25) (layer "F.Cu") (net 5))
 (segment (start 174.005874 105.965874) (end 175.49 107.45) (width 0.25) (layer "F.Cu") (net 5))
 (segment (start 174.574888 100.501634) (end 174.574888 100.941692) (width 0.25) (layer "F.Cu") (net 5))
 (segment (start 177.604506 99.182074) (end 175.844888 97.422456) (width 0.25) (layer "F.Cu") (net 3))
 (segment (start 175.844888 97.422456) (end 175.844888 95.421634) (width 0.25) (layer "F.Cu") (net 3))
 (via (at 177.604506 99.182074) (size 0.8) (drill 0.4) (layers "F.Cu" "B.Cu") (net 3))
 (segment (start 181.745 106.275) (end 180.57 107.45) (width 0.25) (layer "B.Cu") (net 3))
 (segment (start 181.745 103.322568) (end 181.745 106.275) (width 0.25) (layer "B.Cu") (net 3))
 (segment (start 177.604506 99.182074) (end 181.745 103.322568) (width 0.25) (layer "B.Cu") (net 3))
 (segment (start 178.512838 102.467947) (end 178.972388 102.008397) (width 0.25) (layer "F.Cu") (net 2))
 (segment (start 177.114888 97.422456) (end 177.114888 95.421634) (width 0.25) (layer "F.Cu") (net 2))
 (segment (start 178.972388 102.008397) (end 178.972388 99.279956) (width 0.25) (layer "F.Cu") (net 2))
 (segment (start 178.972388 99.279956) (end 177.114888 97.422456) (width 0.25) (layer "F.Cu") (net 2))
 (via (at 178.512838 102.467947) (size 0.8) (drill 0.4) (layers "F.Cu" "B.Cu") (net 2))
 (segment (start 179.395 106.085) (end 178.03 107.45) (width 0.25) (layer "B.Cu") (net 2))
 (segment (start 178.512838 102.467947) (end 179.395 103.350109) (width 0.25) (layer "B.Cu") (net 2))
 (segment (start 179.395 103.350109) (end 179.395 106.085) (width 0.25) (layer "B.Cu") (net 2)))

